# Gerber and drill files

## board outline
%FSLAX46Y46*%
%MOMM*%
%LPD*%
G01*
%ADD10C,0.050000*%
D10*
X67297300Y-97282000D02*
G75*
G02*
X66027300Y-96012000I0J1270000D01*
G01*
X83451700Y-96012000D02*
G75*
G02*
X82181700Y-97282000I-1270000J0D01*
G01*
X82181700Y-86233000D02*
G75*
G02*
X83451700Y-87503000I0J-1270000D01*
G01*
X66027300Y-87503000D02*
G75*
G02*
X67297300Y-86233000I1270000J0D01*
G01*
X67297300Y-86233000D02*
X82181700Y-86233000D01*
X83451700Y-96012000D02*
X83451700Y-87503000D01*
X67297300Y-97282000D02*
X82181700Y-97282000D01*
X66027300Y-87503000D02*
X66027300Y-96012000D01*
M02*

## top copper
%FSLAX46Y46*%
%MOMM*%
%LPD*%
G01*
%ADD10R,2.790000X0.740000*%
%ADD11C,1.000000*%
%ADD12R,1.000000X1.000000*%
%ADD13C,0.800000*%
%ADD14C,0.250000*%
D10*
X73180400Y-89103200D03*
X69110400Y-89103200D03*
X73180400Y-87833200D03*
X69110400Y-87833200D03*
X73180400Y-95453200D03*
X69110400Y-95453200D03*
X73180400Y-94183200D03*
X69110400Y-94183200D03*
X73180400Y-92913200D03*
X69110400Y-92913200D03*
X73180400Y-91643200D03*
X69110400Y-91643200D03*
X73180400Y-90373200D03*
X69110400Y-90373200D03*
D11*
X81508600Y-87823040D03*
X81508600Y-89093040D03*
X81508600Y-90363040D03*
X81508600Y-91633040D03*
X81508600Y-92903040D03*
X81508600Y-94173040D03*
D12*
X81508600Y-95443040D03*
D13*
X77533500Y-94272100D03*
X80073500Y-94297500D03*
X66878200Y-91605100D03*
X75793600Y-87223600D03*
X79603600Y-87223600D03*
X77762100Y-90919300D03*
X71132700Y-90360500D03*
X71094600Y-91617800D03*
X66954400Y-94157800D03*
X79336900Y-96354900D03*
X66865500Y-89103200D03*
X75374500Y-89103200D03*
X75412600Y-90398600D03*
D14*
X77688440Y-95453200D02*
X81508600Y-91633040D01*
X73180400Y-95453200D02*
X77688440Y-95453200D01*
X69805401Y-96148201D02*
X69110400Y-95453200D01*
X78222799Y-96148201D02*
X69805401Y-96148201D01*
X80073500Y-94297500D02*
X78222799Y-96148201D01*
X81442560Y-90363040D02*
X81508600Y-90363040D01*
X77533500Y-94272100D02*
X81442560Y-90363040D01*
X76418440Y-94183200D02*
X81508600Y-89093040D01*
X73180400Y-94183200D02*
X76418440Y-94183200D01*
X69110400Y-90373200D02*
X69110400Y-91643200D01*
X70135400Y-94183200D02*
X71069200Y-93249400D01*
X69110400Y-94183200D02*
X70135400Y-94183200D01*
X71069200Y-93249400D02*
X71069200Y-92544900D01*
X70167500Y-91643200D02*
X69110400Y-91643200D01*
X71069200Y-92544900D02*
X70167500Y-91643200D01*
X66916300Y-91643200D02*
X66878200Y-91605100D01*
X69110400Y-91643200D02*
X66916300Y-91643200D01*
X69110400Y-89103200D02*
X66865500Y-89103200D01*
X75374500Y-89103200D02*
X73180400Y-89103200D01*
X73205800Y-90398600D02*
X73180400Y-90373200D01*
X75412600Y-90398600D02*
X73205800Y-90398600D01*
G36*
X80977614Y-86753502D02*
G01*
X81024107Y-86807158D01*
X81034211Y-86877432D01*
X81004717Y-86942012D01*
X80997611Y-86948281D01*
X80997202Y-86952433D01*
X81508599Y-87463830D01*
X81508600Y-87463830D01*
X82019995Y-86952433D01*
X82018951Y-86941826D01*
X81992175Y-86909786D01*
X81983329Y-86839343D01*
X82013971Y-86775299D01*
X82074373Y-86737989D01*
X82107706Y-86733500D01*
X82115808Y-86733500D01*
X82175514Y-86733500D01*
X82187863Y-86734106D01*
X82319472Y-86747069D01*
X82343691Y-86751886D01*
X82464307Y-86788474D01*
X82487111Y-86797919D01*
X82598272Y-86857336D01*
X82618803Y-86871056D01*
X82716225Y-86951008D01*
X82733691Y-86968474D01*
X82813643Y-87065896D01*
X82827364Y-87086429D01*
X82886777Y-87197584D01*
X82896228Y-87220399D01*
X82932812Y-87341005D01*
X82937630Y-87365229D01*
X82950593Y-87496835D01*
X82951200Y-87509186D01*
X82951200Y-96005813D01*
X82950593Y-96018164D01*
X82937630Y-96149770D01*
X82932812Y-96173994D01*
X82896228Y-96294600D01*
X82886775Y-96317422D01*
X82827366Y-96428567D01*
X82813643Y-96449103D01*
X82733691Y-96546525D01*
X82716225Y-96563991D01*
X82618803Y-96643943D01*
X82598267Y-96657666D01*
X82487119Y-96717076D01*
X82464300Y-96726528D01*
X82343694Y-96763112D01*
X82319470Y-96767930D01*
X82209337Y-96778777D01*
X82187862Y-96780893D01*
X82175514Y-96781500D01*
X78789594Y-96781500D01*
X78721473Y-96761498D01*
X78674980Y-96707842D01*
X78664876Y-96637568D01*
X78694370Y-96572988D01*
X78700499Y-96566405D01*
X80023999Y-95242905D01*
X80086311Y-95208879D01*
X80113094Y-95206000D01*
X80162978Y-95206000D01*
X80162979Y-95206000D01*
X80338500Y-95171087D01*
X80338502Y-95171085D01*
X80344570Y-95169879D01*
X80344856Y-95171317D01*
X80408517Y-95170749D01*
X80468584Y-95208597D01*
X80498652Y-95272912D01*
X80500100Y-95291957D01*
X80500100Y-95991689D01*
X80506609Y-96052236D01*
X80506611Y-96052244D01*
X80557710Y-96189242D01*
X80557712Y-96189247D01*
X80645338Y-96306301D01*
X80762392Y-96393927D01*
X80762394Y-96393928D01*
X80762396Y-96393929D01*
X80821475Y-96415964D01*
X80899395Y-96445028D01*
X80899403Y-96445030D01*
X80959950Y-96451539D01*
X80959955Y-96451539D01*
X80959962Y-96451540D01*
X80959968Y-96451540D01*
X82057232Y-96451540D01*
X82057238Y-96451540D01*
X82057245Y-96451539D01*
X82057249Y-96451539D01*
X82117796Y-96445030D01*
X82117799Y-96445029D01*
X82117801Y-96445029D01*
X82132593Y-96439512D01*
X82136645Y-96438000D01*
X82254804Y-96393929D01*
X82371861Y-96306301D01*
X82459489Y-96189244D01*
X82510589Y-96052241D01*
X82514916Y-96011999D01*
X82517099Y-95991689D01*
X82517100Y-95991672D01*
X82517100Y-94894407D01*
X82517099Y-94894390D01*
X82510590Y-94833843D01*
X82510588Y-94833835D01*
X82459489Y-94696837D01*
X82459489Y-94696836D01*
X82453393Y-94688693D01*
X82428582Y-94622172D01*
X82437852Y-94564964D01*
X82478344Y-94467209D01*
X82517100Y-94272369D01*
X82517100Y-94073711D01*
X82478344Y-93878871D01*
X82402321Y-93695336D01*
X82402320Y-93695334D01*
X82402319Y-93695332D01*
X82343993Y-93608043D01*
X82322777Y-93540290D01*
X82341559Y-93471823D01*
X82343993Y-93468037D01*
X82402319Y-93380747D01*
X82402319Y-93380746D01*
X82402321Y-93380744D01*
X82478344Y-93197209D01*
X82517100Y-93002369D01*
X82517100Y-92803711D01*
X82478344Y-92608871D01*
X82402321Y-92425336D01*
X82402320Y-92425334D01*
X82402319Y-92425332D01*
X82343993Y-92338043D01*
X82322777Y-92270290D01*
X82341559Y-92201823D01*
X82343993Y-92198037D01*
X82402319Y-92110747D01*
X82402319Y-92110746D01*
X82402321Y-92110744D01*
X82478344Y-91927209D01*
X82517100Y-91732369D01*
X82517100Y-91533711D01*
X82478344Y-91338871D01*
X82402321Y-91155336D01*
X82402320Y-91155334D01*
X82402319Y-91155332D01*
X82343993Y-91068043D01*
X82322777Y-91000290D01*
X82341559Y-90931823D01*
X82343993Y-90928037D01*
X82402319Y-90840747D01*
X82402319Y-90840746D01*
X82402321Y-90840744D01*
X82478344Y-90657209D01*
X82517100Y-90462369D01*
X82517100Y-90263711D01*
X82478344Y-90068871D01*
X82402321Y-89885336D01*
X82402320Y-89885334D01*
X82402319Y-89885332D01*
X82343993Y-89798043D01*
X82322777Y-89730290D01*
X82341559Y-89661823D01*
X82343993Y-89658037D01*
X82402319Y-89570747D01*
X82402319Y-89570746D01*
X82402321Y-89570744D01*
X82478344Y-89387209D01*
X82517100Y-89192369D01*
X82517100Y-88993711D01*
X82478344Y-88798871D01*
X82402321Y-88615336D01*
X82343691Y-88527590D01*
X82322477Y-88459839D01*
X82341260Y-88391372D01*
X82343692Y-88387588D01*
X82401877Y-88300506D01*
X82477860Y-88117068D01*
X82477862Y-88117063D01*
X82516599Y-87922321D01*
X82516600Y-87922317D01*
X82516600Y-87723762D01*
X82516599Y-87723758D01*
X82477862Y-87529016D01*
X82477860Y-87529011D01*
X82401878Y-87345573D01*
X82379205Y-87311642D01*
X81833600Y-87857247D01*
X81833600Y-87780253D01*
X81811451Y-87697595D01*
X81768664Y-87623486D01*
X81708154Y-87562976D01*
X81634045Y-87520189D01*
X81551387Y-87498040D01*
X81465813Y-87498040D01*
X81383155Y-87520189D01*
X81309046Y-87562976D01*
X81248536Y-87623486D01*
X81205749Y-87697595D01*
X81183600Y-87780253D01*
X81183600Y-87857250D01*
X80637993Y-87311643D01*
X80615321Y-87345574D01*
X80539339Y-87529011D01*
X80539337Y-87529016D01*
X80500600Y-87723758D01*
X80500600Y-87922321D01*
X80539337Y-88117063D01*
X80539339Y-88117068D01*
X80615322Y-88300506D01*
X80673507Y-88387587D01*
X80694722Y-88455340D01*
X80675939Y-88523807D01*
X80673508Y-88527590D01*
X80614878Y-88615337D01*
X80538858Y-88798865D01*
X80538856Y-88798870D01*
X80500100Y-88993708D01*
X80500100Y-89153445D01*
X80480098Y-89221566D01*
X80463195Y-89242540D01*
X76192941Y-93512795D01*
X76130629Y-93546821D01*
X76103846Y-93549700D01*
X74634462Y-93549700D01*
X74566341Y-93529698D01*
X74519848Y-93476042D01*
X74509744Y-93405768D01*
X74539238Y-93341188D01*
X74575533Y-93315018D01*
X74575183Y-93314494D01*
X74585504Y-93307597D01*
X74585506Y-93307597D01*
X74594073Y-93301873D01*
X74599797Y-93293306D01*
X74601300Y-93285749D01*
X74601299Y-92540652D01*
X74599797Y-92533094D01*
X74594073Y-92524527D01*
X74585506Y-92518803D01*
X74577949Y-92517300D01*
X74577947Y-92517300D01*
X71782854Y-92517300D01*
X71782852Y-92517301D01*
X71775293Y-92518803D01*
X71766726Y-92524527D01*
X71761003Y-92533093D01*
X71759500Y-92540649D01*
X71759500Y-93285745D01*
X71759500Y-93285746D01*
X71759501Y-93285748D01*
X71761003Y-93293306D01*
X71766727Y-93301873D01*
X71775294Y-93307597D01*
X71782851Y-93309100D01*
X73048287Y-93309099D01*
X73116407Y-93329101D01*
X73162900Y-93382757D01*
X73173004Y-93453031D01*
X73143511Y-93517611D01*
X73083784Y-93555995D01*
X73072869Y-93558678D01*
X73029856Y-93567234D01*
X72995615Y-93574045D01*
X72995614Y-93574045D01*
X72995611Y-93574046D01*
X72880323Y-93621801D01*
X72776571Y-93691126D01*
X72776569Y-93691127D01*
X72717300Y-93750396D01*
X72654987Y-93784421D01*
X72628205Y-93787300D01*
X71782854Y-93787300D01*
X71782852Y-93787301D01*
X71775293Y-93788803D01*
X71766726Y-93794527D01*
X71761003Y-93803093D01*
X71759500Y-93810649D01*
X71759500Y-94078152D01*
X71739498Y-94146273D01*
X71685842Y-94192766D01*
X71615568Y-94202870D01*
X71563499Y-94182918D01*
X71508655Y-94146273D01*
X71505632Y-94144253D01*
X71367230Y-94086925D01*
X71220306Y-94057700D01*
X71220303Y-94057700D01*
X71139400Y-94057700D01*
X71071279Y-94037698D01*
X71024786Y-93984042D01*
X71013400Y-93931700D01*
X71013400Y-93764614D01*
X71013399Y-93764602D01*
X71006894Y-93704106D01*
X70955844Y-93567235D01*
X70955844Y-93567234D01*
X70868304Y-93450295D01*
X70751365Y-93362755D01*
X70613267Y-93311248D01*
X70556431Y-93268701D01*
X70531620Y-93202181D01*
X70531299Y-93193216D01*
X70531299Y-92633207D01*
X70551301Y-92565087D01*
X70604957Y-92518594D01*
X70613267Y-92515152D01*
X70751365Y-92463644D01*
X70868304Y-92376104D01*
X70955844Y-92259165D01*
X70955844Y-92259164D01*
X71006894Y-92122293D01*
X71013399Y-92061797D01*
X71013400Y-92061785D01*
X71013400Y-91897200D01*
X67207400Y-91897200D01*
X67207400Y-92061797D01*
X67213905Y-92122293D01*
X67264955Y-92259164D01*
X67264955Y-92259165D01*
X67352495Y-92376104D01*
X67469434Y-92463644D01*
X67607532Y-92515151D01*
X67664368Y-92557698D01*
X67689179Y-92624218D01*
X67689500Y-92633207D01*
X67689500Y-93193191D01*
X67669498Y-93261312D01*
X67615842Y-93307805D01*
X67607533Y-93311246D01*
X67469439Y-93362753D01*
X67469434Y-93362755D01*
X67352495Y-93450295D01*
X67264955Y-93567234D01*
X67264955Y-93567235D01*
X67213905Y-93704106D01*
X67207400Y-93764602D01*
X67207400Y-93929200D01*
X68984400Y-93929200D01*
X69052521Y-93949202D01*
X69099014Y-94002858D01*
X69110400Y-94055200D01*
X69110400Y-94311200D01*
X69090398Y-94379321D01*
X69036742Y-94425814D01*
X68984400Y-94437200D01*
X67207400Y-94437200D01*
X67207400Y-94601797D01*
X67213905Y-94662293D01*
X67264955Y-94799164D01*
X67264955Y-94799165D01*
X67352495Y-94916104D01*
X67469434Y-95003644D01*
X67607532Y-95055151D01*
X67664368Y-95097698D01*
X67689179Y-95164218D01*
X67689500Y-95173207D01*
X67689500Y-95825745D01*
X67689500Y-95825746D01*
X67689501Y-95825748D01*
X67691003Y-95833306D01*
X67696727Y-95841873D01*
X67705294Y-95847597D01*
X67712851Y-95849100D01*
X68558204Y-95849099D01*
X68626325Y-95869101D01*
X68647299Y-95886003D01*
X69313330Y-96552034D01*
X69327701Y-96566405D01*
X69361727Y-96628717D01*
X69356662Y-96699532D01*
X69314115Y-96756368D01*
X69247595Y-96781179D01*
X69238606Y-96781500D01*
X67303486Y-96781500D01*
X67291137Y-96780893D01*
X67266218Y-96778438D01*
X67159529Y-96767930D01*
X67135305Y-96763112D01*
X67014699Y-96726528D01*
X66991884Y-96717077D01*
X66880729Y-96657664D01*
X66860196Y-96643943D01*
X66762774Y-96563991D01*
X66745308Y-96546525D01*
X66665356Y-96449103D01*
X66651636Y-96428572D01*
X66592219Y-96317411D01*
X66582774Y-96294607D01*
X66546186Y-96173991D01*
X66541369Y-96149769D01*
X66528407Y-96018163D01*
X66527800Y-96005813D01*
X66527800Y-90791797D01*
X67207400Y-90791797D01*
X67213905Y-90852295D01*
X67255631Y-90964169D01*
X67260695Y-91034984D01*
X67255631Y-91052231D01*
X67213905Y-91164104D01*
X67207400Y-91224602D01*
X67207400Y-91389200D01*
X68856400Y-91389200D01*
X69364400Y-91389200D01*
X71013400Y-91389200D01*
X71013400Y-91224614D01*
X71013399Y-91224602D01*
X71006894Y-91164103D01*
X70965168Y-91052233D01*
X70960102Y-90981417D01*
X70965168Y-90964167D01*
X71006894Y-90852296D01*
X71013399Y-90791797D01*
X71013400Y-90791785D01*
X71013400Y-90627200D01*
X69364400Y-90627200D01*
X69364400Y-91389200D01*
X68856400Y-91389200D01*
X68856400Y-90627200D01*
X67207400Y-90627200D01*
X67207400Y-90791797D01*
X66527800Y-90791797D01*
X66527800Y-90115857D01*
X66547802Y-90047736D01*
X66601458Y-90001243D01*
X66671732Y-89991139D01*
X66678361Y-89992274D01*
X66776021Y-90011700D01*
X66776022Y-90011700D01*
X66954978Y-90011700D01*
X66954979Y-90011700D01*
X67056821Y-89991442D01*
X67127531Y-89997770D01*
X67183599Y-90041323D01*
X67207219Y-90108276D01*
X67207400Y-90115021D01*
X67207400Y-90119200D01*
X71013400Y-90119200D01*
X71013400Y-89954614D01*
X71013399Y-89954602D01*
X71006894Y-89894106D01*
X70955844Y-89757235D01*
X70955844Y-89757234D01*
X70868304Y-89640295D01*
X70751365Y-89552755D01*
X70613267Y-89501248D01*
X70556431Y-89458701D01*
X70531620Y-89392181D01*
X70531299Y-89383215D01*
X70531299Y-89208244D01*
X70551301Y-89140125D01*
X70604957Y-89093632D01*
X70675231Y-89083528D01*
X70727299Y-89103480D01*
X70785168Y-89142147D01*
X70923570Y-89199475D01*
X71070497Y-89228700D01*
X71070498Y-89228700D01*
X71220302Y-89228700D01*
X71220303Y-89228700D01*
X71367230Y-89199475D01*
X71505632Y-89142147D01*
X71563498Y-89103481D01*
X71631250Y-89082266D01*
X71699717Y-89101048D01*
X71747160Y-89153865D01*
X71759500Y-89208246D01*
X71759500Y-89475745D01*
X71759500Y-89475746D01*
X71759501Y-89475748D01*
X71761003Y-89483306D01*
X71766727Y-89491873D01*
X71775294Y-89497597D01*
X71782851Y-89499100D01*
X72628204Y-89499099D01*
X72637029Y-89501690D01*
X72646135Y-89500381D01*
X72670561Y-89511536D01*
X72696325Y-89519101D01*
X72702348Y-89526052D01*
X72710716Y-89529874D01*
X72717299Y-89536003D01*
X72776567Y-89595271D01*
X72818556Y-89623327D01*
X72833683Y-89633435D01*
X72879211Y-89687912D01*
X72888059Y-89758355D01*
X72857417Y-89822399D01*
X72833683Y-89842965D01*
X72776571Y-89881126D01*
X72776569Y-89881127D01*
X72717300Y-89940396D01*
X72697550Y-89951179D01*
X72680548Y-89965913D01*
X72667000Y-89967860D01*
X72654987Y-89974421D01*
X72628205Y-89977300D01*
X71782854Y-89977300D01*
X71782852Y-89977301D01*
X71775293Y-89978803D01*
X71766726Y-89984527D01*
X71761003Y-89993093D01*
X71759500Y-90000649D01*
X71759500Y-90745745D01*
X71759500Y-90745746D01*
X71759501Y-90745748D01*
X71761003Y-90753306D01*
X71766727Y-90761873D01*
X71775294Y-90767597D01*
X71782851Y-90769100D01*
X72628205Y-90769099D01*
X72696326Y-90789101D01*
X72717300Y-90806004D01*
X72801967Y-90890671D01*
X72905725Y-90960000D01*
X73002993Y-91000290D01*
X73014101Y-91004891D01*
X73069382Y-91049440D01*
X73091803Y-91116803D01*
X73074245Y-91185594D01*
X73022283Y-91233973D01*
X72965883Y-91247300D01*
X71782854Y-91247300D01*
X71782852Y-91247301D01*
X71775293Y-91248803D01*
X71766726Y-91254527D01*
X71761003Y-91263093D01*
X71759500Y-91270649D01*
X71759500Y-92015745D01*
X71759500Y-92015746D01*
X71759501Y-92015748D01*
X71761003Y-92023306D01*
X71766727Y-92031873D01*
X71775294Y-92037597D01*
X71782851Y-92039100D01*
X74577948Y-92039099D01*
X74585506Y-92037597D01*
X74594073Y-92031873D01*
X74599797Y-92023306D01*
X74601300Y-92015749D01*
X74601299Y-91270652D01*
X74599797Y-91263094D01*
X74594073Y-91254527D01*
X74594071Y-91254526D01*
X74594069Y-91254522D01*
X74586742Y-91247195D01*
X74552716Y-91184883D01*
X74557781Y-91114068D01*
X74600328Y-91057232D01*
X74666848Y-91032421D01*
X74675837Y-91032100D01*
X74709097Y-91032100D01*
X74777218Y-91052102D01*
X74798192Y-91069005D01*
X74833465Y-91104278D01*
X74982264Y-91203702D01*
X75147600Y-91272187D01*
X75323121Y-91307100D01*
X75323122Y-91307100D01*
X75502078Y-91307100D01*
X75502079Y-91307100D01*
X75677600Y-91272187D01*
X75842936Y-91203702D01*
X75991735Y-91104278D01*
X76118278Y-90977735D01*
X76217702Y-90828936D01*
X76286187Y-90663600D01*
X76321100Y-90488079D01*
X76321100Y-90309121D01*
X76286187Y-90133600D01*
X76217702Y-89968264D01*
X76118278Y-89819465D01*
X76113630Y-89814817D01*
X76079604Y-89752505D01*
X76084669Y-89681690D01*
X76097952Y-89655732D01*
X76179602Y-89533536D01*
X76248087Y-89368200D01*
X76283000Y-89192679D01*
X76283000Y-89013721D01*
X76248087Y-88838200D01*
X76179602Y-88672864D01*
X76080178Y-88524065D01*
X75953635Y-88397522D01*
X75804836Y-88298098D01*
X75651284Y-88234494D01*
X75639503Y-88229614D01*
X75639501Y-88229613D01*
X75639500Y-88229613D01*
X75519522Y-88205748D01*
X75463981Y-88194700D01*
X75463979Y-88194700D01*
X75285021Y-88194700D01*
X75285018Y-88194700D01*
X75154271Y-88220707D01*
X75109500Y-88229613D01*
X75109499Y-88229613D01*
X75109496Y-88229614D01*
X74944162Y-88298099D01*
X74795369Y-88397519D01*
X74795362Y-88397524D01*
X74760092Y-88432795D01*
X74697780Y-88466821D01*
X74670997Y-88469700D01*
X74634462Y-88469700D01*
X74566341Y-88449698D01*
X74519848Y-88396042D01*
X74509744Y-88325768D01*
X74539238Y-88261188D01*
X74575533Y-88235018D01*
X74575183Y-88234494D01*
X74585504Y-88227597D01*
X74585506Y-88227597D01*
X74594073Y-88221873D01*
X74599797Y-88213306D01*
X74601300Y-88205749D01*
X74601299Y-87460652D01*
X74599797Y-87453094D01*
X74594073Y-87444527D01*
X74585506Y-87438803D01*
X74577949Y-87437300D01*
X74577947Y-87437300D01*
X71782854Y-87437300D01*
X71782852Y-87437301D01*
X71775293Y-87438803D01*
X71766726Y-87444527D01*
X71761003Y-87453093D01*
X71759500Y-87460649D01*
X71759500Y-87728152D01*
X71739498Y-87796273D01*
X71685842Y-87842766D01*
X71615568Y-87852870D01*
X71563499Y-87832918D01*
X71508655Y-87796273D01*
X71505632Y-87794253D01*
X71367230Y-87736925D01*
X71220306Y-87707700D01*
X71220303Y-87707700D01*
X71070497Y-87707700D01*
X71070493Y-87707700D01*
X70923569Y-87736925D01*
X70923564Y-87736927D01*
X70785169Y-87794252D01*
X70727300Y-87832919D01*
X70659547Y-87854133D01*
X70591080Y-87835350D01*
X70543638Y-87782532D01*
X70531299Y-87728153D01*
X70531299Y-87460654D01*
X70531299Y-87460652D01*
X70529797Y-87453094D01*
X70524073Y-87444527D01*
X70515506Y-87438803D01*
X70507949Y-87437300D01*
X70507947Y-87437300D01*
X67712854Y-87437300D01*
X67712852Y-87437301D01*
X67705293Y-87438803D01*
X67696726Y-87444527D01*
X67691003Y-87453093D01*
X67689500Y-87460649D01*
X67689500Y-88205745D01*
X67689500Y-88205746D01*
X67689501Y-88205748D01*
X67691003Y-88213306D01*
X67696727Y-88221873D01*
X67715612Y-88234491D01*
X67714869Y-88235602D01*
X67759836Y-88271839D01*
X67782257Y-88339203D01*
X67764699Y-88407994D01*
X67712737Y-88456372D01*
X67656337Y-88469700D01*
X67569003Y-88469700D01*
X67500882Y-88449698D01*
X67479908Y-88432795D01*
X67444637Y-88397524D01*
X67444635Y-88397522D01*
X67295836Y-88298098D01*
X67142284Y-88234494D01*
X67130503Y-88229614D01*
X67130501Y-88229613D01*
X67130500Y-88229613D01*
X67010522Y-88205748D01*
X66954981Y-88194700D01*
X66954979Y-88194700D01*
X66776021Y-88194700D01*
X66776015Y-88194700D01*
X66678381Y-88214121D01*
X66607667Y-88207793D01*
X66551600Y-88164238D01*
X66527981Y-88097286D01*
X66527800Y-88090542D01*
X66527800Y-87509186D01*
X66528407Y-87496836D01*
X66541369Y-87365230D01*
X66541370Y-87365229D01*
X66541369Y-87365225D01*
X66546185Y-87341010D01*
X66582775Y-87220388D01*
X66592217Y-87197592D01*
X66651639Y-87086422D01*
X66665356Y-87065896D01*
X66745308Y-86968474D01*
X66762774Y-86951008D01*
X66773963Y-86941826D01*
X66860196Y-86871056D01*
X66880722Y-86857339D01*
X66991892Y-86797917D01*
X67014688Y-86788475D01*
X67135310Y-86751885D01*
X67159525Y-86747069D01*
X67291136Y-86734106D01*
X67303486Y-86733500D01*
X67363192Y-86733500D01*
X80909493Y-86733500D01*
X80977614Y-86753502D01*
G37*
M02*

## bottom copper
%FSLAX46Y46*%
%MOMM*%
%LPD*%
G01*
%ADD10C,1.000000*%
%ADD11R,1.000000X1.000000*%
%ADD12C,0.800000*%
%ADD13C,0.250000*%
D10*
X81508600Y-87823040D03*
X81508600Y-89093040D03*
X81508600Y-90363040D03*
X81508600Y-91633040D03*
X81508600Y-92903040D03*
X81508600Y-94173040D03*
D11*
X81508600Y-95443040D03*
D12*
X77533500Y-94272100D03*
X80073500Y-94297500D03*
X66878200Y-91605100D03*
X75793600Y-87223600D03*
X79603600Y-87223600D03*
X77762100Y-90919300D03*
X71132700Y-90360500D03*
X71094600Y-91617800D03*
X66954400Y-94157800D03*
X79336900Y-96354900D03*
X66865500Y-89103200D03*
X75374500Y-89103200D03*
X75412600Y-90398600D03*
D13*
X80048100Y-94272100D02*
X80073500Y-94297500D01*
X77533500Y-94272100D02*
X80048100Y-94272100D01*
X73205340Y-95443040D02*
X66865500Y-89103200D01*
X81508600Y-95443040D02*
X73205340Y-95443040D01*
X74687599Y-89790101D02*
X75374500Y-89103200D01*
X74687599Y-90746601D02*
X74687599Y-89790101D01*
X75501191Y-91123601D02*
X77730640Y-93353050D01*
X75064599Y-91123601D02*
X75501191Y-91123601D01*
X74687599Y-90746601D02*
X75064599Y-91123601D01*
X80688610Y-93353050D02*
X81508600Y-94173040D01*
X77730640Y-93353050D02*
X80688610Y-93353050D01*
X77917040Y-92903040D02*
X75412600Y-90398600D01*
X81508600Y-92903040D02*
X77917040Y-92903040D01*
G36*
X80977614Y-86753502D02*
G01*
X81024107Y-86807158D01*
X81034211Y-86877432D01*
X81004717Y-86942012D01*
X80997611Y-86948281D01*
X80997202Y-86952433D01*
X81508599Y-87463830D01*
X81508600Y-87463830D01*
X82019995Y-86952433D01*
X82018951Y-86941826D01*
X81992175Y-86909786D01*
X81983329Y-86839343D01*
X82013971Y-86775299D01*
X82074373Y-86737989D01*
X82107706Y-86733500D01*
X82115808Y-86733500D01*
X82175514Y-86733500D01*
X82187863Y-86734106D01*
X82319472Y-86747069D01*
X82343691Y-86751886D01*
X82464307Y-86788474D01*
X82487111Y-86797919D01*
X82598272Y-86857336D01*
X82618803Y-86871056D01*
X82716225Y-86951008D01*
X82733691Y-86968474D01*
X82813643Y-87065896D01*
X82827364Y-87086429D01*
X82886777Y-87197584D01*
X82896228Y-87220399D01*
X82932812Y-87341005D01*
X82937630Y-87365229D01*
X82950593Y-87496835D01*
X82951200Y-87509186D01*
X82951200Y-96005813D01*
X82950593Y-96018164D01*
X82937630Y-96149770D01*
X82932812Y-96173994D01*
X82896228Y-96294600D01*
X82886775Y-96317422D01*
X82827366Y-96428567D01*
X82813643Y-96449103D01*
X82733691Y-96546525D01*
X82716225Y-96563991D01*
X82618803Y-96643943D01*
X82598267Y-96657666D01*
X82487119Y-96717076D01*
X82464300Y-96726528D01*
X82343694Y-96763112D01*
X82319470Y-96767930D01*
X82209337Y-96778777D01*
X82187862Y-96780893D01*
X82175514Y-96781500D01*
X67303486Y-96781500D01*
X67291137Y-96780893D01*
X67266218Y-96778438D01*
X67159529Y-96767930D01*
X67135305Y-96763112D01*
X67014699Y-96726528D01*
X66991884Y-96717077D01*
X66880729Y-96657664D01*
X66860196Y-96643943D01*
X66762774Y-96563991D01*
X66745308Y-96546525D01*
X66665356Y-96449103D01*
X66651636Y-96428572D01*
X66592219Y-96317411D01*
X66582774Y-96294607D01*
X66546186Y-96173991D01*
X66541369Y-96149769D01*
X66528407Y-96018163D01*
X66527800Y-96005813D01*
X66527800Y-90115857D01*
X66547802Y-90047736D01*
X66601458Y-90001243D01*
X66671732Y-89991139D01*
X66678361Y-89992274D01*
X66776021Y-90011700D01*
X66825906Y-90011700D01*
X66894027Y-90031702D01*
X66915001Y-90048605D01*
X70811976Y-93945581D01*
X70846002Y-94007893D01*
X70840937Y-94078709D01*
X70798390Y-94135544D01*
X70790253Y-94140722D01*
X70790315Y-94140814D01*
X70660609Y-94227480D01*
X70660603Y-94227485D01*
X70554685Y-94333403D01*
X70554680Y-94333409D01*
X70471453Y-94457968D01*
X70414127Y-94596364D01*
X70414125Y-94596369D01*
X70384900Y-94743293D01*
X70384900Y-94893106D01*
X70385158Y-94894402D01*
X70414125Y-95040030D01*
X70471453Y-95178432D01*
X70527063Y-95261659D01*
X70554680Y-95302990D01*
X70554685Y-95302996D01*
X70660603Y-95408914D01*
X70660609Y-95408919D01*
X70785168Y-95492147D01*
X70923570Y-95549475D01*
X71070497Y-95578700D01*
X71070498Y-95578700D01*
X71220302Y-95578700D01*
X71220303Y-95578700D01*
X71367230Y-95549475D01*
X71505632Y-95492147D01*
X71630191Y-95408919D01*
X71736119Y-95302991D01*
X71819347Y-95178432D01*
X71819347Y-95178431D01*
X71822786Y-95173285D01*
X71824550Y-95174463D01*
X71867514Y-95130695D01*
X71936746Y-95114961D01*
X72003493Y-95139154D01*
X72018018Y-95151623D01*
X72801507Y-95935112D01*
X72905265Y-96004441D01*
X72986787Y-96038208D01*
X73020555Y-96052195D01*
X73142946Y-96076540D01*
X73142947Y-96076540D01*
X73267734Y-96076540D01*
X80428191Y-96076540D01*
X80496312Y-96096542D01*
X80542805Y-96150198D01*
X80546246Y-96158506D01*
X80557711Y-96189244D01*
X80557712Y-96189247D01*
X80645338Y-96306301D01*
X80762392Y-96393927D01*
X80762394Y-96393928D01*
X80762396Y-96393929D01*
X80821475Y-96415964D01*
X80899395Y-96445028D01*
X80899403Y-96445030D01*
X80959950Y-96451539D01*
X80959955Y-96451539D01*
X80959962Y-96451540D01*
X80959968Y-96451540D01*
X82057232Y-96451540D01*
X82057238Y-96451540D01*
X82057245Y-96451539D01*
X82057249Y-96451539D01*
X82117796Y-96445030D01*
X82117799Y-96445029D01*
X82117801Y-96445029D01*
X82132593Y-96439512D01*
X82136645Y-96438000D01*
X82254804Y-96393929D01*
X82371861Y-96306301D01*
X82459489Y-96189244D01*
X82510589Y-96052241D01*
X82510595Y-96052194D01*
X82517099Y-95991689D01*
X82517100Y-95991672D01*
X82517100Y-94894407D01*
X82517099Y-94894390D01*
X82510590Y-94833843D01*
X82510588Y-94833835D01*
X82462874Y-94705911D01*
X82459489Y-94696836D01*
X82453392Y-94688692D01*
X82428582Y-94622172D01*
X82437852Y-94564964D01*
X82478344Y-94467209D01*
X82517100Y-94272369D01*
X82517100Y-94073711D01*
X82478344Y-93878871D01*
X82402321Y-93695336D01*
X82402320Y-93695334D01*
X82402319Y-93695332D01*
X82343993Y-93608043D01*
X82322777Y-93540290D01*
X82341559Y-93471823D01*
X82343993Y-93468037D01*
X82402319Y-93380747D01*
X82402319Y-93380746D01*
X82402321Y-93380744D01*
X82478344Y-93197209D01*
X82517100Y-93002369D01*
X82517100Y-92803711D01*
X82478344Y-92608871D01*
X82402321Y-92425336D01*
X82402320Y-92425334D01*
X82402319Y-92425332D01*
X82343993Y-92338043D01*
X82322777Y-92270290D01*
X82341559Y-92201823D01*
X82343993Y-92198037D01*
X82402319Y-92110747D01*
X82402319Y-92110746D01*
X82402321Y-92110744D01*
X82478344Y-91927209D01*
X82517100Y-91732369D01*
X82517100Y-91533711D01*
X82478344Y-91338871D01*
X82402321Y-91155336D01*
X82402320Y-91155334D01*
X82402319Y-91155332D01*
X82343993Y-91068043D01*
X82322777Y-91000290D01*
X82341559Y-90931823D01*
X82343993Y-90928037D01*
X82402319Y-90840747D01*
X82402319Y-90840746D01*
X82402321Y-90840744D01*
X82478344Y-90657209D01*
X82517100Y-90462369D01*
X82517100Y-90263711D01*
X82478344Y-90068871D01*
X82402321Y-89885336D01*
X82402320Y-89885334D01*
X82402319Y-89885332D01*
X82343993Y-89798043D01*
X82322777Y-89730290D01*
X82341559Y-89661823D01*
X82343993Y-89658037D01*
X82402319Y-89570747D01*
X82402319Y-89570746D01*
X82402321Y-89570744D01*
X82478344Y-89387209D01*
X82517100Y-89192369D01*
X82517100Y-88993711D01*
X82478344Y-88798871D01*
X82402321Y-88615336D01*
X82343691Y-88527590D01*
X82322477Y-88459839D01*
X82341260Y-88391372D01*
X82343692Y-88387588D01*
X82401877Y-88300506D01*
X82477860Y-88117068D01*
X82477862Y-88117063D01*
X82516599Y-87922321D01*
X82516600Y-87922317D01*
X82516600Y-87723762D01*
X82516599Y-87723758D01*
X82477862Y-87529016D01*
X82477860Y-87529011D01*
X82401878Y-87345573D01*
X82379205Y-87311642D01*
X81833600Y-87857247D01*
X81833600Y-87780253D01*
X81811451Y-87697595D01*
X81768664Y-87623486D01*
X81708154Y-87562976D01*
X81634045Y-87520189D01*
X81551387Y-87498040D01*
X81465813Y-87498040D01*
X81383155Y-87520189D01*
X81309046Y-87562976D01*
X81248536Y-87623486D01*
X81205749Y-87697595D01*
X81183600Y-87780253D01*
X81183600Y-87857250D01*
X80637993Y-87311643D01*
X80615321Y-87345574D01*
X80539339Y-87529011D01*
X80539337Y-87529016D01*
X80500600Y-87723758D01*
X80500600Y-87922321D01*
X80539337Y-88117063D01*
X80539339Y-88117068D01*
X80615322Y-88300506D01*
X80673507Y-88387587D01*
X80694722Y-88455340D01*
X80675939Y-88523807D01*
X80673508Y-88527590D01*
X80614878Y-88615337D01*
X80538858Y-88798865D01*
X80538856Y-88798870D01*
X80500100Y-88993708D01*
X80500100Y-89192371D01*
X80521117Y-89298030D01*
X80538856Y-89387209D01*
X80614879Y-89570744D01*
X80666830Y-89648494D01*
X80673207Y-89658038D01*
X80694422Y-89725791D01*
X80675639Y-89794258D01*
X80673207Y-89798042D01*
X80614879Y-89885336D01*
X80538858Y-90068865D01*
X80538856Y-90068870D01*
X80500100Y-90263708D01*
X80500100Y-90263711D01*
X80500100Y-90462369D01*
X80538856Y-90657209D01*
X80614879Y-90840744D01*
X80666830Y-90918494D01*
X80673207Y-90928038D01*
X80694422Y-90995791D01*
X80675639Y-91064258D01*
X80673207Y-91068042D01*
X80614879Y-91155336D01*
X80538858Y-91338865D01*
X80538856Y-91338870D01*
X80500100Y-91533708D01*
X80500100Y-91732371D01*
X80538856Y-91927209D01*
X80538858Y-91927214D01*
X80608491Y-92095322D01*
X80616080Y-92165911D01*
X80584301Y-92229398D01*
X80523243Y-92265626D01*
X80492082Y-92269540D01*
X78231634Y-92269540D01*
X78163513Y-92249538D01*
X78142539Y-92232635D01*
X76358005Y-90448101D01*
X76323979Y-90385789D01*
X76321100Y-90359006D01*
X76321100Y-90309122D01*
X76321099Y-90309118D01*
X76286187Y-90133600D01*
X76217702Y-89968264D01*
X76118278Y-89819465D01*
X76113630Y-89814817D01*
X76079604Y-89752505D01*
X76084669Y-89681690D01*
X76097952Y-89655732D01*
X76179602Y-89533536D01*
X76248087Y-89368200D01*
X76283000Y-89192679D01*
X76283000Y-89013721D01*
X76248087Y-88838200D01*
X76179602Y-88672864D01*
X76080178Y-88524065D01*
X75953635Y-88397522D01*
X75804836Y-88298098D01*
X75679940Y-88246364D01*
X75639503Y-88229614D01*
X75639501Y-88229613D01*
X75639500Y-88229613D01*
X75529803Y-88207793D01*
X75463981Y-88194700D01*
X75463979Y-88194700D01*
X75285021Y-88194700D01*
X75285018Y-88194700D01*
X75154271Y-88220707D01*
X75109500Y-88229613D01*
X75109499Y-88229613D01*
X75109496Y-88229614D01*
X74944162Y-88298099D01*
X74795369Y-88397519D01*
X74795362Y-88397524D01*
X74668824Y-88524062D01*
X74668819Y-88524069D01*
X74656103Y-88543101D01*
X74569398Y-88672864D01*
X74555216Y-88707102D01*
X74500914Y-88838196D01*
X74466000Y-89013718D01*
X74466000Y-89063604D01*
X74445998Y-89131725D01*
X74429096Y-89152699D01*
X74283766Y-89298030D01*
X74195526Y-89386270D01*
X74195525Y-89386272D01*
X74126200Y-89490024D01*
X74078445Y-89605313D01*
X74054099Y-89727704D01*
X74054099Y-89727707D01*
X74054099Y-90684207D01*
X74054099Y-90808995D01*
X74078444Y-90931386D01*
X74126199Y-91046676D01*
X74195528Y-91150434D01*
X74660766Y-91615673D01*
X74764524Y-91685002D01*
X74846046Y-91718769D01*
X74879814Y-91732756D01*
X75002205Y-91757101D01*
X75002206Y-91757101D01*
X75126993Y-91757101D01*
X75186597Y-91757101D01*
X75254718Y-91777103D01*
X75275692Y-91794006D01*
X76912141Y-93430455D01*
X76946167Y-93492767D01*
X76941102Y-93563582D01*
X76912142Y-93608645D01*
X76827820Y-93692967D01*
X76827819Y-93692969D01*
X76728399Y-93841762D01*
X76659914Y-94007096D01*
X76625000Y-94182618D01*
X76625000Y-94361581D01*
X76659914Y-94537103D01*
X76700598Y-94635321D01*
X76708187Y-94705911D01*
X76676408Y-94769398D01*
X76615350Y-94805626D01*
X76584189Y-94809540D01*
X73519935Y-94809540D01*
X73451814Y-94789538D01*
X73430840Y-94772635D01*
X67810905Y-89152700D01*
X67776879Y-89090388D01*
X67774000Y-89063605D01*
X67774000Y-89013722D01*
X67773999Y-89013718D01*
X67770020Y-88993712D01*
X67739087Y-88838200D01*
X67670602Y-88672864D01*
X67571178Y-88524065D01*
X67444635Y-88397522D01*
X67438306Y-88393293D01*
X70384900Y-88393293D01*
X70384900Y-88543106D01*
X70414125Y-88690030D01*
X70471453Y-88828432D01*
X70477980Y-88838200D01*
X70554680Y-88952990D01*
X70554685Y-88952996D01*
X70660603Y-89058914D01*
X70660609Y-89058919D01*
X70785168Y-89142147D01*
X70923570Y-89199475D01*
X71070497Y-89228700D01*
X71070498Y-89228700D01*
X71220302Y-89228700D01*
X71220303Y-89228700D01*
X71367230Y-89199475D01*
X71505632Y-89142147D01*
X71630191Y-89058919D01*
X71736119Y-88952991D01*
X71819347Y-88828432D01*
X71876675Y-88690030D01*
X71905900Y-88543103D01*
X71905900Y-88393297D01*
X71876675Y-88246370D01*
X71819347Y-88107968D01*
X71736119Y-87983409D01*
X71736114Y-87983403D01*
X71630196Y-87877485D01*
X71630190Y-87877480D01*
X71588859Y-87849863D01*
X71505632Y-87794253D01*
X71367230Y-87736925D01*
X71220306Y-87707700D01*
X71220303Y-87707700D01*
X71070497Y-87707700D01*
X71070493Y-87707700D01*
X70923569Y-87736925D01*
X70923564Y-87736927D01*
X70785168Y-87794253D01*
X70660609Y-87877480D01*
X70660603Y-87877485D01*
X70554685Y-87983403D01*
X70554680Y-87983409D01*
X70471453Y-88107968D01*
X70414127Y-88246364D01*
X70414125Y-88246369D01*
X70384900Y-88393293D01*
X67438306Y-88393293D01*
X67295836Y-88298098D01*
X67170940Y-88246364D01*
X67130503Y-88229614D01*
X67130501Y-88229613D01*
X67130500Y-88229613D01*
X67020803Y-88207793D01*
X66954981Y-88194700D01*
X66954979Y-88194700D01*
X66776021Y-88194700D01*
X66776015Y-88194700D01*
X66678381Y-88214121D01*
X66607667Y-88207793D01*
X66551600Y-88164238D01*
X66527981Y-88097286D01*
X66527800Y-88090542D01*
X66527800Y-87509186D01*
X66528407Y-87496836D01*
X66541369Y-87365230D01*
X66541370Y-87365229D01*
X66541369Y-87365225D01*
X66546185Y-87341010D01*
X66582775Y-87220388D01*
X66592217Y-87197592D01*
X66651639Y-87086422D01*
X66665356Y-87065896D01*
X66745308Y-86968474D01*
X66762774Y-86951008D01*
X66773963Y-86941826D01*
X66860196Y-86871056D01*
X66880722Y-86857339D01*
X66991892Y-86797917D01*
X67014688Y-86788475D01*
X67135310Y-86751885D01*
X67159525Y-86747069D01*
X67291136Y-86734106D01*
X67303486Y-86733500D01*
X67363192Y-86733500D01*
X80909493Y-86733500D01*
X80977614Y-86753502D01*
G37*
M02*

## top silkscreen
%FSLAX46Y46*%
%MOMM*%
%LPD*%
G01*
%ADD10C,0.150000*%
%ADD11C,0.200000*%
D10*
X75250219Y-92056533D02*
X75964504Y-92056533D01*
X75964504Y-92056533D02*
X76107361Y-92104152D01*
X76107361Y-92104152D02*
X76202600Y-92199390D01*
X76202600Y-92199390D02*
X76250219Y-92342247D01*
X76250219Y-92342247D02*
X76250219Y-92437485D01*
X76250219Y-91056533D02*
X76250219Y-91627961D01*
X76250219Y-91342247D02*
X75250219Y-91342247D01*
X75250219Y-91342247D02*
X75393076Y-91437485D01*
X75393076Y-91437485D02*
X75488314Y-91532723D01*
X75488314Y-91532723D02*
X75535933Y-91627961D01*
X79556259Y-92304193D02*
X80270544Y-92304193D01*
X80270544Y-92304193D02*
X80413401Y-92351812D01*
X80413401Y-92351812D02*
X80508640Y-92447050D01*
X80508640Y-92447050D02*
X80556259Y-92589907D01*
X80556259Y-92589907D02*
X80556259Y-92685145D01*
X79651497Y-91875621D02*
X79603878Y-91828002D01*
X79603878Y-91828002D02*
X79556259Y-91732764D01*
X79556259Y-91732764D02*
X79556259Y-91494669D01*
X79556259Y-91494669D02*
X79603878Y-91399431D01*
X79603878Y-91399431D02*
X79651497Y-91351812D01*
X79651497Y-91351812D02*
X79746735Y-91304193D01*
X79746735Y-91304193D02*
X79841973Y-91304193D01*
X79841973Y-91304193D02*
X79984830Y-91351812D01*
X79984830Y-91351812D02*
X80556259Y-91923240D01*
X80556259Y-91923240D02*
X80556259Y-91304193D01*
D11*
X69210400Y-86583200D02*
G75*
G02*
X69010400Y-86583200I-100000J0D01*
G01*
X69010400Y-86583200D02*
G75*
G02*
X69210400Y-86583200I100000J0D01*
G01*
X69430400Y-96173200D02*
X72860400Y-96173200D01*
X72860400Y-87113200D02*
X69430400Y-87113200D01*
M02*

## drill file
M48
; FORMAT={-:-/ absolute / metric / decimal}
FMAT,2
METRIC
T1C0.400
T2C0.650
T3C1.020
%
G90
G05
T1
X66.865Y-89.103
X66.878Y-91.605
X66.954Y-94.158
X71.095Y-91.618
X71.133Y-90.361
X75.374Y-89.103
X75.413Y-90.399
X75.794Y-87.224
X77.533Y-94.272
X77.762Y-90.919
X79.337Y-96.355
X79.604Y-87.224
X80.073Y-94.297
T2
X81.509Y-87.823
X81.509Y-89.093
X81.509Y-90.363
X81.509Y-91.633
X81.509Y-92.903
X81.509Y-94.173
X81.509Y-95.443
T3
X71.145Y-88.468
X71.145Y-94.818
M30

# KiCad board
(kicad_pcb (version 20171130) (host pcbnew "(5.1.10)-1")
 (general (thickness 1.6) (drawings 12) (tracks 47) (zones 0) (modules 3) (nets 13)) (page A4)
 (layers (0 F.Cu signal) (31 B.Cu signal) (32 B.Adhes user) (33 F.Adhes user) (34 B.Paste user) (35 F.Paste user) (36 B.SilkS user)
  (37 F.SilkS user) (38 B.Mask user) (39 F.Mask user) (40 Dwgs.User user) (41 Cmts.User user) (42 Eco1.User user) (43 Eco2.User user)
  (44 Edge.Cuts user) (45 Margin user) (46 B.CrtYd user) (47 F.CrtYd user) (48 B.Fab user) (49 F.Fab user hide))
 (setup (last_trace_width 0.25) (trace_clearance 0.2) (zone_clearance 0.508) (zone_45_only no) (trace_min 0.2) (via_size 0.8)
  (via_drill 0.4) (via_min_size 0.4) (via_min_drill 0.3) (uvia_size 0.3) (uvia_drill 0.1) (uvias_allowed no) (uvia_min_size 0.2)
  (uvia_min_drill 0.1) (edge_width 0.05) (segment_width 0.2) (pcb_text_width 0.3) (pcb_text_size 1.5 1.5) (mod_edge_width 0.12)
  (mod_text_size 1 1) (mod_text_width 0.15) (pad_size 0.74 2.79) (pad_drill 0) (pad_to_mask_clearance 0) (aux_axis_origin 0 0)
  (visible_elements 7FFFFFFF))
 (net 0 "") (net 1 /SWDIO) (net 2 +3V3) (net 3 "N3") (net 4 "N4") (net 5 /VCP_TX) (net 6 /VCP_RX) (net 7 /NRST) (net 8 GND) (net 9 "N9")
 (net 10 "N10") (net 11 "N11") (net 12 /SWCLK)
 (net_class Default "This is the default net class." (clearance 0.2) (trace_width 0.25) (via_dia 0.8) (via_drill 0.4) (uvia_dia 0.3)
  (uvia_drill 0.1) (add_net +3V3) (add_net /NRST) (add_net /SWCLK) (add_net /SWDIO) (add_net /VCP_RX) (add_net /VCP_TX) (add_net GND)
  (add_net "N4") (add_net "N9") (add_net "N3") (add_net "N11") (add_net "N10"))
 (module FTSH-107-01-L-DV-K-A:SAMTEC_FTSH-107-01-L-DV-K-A (layer F.Cu) (at 71.1454 91.6432 270) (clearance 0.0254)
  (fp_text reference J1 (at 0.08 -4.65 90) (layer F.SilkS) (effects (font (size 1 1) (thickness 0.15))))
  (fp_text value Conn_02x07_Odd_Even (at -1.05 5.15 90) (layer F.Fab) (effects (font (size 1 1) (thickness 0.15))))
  (fp_circle (center -5.06 2.035) (end -4.96 2.035) (layer F.SilkS) (width 0.2))
  (fp_line (start 4.53 1.715) (end 4.53 -1.715) (layer F.SilkS) (width 0.2))
  (fp_line (start -4.53 -1.715) (end -4.53 1.715) (layer F.SilkS) (width 0.2))
  (pad 4 smd rect (at -2.54 -2.035 270) (size 0.74 2.79) (layers F.Cu F.Paste F.Mask) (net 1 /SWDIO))
  (pad 3 smd rect (at -2.54 2.035 270) (size 0.74 2.79) (layers F.Cu F.Paste F.Mask) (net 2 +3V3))
  (pad 2 smd rect (at -3.81 -2.035 270) (size 0.74 2.79) (layers F.Cu F.Paste F.Mask) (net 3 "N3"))
  (pad 1 smd rect (at -3.81 2.035 270) (size 0.74 2.79) (layers F.Cu F.Paste F.Mask) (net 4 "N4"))
  (pad None np_thru_hole circle (at -3.175 0 270) (size 1.02 1.02) (drill 1.02) (layers *.Cu *.Mask))
  (pad None np_thru_hole circle (at 3.175 0 270) (size 1.02 1.02) (drill 1.02) (layers *.Cu *.Mask))
  (pad 14 smd rect (at 3.81 -2.035 270) (size 0.74 2.79) (layers F.Cu F.Paste F.Mask) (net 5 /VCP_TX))
  (pad 13 smd rect (at 3.81 2.035 270) (size 0.74 2.79) (layers F.Cu F.Paste F.Mask) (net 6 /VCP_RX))
  (pad 12 smd rect (at 2.54 -2.035 270) (size 0.74 2.79) (layers F.Cu F.Paste F.Mask) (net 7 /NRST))
  (pad 11 smd rect (at 2.54 2.035 270) (size 0.74 2.79) (layers F.Cu F.Paste F.Mask) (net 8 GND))
  (pad 10 smd rect (at 1.27 -2.035 270) (size 0.74 2.79) (layers F.Cu F.Paste F.Mask) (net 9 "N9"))
  (pad 9 smd rect (at 1.27 2.035 270) (size 0.74 2.79) (layers F.Cu F.Paste F.Mask) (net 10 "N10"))
  (pad 8 smd rect (at 0 -2.035 270) (size 0.74 2.79) (layers F.Cu F.Paste F.Mask) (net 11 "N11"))
  (pad 7 smd rect (at 0 2.035 270) (size 0.74 2.79) (layers F.Cu F.Paste F.Mask) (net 8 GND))
  (pad 6 smd rect (at -1.27 -2.035 270) (size 0.74 2.79) (layers F.Cu F.Paste F.Mask) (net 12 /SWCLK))
  (pad 5 smd rect (at -1.27 2.035 270) (size 0.74 2.79) (layers F.Cu F.Paste F.Mask) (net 8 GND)))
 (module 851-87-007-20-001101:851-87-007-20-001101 (layer F.Cu) (at 81.5086 95.4278 90)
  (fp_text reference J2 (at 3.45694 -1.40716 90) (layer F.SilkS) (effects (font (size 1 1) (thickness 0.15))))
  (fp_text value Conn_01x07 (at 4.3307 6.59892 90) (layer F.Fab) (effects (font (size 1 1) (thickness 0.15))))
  (pad 7 thru_hole circle (at 7.60476 0 90) (size 1 1) (drill 0.65) (layers *.Cu *.Mask) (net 8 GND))
  (pad 6 thru_hole circle (at 6.33476 0 90) (size 1 1) (drill 0.65) (layers *.Cu *.Mask) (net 7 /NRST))
  (pad 5 thru_hole circle (at 5.06476 0 90) (size 1 1) (drill 0.65) (layers *.Cu *.Mask) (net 6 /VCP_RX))
  (pad 4 thru_hole circle (at 3.79476 0 90) (size 1 1) (drill 0.65) (layers *.Cu *.Mask) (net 5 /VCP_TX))
  (pad 3 thru_hole circle (at 2.52476 0 90) (size 1 1) (drill 0.65) (layers *.Cu *.Mask) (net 12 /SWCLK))
  (pad 2 thru_hole circle (at 1.25476 0 90) (size 1 1) (drill 0.65) (layers *.Cu *.Mask) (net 1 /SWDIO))
  (pad 1 thru_hole rect (at -0.01524 0 90) (size 1 1) (drill 0.65) (layers *.Cu *.Mask) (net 2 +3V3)))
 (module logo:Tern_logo (layer B.Cu) (at 71.5899 92.202 180)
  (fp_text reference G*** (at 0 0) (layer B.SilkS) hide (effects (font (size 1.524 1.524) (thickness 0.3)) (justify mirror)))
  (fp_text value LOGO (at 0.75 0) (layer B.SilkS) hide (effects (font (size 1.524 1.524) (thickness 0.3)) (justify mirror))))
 (gr_arc (start 67.2973 96.012) (end 66.0273 96.012) (angle -90) (layer Edge.Cuts) (width 0.05))
 (gr_arc (start 82.1817 96.012) (end 82.1817 97.282) (angle -90) (layer Edge.Cuts) (width 0.05))
 (gr_arc (start 82.1817 87.503) (end 83.4517 87.503) (angle -90) (layer Edge.Cuts) (width 0.05))
 (gr_arc (start 67.2973 87.503) (end 67.2973 86.233) (angle -90) (layer Edge.Cuts) (width 0.05))
 (gr_line (start 67.2973 86.233) (end 82.1817 86.233) (layer Edge.Cuts) (width 0.05))
 (gr_line (start 83.4517 96.012) (end 83.4517 87.503) (layer Edge.Cuts) (width 0.05))
 (gr_line (start 67.2973 97.282) (end 82.1817 97.282) (layer Edge.Cuts) (width 0.05))
 (gr_line (start 66.0273 87.503) (end 66.0273 96.012) (layer Edge.Cuts) (width 0.05))
 (segment (start 77.68844 95.4532) (end 81.5086 91.63304) (width 0.25) (layer F.Cu) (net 5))
 (segment (start 73.1804 95.4532) (end 77.68844 95.4532) (width 0.25) (layer F.Cu) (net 5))
 (via (at 77.5335 94.2721) (size 0.8) (drill 0.4) (layers F.Cu B.Cu) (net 6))
 (via (at 80.0735 94.2975) (size 0.8) (drill 0.4) (layers F.Cu B.Cu) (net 6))
 (segment (start 80.0481 94.2721) (end 80.0735 94.2975) (width 0.25) (layer B.Cu) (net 6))
 (segment (start 77.5335 94.2721) (end 80.0481 94.2721) (width 0.25) (layer B.Cu) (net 6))
 (segment (start 69.805401 96.148201) (end 69.1104 95.4532) (width 0.25) (layer F.Cu) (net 6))
 (segment (start 78.222799 96.148201) (end 69.805401 96.148201) (width 0.25) (layer F.Cu) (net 6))
 (segment (start 80.0735 94.2975) (end 78.222799 96.148201) (width 0.25) (layer F.Cu) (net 6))
 (segment (start 81.44256 90.36304) (end 81.5086 90.36304) (width 0.25) (layer F.Cu) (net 6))
 (segment (start 77.5335 94.2721) (end 81.44256 90.36304) (width 0.25) (layer F.Cu) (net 6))
 (segment (start 76.41844 94.1832) (end 81.5086 89.09304) (width 0.25) (layer F.Cu) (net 7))
 (segment (start 73.1804 94.1832) (end 76.41844 94.1832) (width 0.25) (layer F.Cu) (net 7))
 (segment (start 69.1104 90.3732) (end 69.1104 91.6432) (width 0.25) (layer F.Cu) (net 8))
 (segment (start 70.1354 94.1832) (end 71.0692 93.2494) (width 0.25) (layer F.Cu) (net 8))
 (segment (start 69.1104 94.1832) (end 70.1354 94.1832) (width 0.25) (layer F.Cu) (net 8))
 (segment (start 71.0692 93.2494) (end 71.0692 92.5449) (width 0.25) (layer F.Cu) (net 8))
 (segment (start 70.1675 91.6432) (end 69.1104 91.6432) (width 0.25) (layer F.Cu) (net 8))
 (segment (start 71.0692 92.5449) (end 70.1675 91.6432) (width 0.25) (layer F.Cu) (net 8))
 (via (at 66.8782 91.6051) (size 0.8) (drill 0.4) (layers F.Cu B.Cu) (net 8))
 (segment (start 66.9163 91.6432) (end 66.8782 91.6051) (width 0.25) (layer F.Cu) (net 8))
 (segment (start 69.1104 91.6432) (end 66.9163 91.6432) (width 0.25) (layer F.Cu) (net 8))
 (via (at 75.7936 87.2236) (size 0.8) (drill 0.4) (layers F.Cu B.Cu) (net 8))
 (via (at 79.6036 87.2236) (size 0.8) (drill 0.4) (layers F.Cu B.Cu) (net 8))
 (via (at 77.7621 90.9193) (size 0.8) (drill 0.4) (layers F.Cu B.Cu) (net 8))
 (via (at 71.1327 90.3605) (size 0.8) (drill 0.4) (layers F.Cu B.Cu) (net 8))
 (via (at 71.0946 91.6178) (size 0.8) (drill 0.4) (layers F.Cu B.Cu) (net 8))
 (via (at 66.9544 94.1578) (size 0.8) (drill 0.4) (layers F.Cu B.Cu) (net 8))
 (via (at 79.3369 96.3549) (size 0.8) (drill 0.4) (layers F.Cu B.Cu) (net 8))
 (via (at 66.8655 89.1032) (size 0.8) (drill 0.4) (layers F.Cu B.Cu) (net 2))
 (segment (start 69.1104 89.1032) (end 66.8655 89.1032) (width 0.25) (layer F.Cu) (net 2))
 (segment (start 73.20534 95.44304) (end 66.8655 89.1032) (width 0.25) (layer B.Cu) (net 2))
 (segment (start 81.5086 95.44304) (end 73.20534 95.44304) (width 0.25) (layer B.Cu) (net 2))
 (via (at 75.3745 89.1032) (size 0.8) (drill 0.4) (layers F.Cu B.Cu) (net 1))
 (segment (start 74.687599 89.790101) (end 75.3745 89.1032) (width 0.25) (layer B.Cu) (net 1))
 (segment (start 74.687599 90.746601) (end 74.687599 89.790101) (width 0.25) (layer B.Cu) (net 1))
 (segment (start 75.3745 89.1032) (end 73.1804 89.1032) (width 0.25) (layer F.Cu) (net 1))
 (segment (start 75.501191 91.123601) (end 77.73064 93.35305) (width 0.25) (layer B.Cu) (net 1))
 (segment (start 75.064599 91.123601) (end 75.501191 91.123601) (width 0.25) (layer B.Cu) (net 1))
 (segment (start 74.687599 90.746601) (end 75.064599 91.123601) (width 0.25) (layer B.Cu) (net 1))
 (segment (start 80.68861 93.35305) (end 81.5086 94.17304) (width 0.25) (layer B.Cu) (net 1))
 (segment (start 77.73064 93.35305) (end 80.68861 93.35305) (width 0.25) (layer B.Cu) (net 1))
 (via (at 75.4126 90.3986) (size 0.8) (drill 0.4) (layers F.Cu B.Cu) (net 12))
 (segment (start 77.91704 92.90304) (end 75.4126 90.3986) (width 0.25) (layer B.Cu) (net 12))
 (segment (start 81.5086 92.90304) (end 77.91704 92.90304) (width 0.25) (layer B.Cu) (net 12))
 (segment (start 73.2058 90.3986) (end 73.1804 90.3732) (width 0.25) (layer F.Cu) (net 12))
 (segment (start 75.4126 90.3986) (end 73.2058 90.3986) (width 0.25) (layer F.Cu) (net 12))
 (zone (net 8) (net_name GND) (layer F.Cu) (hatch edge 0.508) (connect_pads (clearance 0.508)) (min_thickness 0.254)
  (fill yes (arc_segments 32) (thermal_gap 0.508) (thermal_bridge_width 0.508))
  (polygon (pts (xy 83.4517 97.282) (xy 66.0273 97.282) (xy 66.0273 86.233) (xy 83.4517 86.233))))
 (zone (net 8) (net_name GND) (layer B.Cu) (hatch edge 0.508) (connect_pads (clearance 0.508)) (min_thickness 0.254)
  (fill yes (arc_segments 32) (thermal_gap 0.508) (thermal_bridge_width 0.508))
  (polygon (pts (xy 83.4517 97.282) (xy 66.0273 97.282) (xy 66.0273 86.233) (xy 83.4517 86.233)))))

